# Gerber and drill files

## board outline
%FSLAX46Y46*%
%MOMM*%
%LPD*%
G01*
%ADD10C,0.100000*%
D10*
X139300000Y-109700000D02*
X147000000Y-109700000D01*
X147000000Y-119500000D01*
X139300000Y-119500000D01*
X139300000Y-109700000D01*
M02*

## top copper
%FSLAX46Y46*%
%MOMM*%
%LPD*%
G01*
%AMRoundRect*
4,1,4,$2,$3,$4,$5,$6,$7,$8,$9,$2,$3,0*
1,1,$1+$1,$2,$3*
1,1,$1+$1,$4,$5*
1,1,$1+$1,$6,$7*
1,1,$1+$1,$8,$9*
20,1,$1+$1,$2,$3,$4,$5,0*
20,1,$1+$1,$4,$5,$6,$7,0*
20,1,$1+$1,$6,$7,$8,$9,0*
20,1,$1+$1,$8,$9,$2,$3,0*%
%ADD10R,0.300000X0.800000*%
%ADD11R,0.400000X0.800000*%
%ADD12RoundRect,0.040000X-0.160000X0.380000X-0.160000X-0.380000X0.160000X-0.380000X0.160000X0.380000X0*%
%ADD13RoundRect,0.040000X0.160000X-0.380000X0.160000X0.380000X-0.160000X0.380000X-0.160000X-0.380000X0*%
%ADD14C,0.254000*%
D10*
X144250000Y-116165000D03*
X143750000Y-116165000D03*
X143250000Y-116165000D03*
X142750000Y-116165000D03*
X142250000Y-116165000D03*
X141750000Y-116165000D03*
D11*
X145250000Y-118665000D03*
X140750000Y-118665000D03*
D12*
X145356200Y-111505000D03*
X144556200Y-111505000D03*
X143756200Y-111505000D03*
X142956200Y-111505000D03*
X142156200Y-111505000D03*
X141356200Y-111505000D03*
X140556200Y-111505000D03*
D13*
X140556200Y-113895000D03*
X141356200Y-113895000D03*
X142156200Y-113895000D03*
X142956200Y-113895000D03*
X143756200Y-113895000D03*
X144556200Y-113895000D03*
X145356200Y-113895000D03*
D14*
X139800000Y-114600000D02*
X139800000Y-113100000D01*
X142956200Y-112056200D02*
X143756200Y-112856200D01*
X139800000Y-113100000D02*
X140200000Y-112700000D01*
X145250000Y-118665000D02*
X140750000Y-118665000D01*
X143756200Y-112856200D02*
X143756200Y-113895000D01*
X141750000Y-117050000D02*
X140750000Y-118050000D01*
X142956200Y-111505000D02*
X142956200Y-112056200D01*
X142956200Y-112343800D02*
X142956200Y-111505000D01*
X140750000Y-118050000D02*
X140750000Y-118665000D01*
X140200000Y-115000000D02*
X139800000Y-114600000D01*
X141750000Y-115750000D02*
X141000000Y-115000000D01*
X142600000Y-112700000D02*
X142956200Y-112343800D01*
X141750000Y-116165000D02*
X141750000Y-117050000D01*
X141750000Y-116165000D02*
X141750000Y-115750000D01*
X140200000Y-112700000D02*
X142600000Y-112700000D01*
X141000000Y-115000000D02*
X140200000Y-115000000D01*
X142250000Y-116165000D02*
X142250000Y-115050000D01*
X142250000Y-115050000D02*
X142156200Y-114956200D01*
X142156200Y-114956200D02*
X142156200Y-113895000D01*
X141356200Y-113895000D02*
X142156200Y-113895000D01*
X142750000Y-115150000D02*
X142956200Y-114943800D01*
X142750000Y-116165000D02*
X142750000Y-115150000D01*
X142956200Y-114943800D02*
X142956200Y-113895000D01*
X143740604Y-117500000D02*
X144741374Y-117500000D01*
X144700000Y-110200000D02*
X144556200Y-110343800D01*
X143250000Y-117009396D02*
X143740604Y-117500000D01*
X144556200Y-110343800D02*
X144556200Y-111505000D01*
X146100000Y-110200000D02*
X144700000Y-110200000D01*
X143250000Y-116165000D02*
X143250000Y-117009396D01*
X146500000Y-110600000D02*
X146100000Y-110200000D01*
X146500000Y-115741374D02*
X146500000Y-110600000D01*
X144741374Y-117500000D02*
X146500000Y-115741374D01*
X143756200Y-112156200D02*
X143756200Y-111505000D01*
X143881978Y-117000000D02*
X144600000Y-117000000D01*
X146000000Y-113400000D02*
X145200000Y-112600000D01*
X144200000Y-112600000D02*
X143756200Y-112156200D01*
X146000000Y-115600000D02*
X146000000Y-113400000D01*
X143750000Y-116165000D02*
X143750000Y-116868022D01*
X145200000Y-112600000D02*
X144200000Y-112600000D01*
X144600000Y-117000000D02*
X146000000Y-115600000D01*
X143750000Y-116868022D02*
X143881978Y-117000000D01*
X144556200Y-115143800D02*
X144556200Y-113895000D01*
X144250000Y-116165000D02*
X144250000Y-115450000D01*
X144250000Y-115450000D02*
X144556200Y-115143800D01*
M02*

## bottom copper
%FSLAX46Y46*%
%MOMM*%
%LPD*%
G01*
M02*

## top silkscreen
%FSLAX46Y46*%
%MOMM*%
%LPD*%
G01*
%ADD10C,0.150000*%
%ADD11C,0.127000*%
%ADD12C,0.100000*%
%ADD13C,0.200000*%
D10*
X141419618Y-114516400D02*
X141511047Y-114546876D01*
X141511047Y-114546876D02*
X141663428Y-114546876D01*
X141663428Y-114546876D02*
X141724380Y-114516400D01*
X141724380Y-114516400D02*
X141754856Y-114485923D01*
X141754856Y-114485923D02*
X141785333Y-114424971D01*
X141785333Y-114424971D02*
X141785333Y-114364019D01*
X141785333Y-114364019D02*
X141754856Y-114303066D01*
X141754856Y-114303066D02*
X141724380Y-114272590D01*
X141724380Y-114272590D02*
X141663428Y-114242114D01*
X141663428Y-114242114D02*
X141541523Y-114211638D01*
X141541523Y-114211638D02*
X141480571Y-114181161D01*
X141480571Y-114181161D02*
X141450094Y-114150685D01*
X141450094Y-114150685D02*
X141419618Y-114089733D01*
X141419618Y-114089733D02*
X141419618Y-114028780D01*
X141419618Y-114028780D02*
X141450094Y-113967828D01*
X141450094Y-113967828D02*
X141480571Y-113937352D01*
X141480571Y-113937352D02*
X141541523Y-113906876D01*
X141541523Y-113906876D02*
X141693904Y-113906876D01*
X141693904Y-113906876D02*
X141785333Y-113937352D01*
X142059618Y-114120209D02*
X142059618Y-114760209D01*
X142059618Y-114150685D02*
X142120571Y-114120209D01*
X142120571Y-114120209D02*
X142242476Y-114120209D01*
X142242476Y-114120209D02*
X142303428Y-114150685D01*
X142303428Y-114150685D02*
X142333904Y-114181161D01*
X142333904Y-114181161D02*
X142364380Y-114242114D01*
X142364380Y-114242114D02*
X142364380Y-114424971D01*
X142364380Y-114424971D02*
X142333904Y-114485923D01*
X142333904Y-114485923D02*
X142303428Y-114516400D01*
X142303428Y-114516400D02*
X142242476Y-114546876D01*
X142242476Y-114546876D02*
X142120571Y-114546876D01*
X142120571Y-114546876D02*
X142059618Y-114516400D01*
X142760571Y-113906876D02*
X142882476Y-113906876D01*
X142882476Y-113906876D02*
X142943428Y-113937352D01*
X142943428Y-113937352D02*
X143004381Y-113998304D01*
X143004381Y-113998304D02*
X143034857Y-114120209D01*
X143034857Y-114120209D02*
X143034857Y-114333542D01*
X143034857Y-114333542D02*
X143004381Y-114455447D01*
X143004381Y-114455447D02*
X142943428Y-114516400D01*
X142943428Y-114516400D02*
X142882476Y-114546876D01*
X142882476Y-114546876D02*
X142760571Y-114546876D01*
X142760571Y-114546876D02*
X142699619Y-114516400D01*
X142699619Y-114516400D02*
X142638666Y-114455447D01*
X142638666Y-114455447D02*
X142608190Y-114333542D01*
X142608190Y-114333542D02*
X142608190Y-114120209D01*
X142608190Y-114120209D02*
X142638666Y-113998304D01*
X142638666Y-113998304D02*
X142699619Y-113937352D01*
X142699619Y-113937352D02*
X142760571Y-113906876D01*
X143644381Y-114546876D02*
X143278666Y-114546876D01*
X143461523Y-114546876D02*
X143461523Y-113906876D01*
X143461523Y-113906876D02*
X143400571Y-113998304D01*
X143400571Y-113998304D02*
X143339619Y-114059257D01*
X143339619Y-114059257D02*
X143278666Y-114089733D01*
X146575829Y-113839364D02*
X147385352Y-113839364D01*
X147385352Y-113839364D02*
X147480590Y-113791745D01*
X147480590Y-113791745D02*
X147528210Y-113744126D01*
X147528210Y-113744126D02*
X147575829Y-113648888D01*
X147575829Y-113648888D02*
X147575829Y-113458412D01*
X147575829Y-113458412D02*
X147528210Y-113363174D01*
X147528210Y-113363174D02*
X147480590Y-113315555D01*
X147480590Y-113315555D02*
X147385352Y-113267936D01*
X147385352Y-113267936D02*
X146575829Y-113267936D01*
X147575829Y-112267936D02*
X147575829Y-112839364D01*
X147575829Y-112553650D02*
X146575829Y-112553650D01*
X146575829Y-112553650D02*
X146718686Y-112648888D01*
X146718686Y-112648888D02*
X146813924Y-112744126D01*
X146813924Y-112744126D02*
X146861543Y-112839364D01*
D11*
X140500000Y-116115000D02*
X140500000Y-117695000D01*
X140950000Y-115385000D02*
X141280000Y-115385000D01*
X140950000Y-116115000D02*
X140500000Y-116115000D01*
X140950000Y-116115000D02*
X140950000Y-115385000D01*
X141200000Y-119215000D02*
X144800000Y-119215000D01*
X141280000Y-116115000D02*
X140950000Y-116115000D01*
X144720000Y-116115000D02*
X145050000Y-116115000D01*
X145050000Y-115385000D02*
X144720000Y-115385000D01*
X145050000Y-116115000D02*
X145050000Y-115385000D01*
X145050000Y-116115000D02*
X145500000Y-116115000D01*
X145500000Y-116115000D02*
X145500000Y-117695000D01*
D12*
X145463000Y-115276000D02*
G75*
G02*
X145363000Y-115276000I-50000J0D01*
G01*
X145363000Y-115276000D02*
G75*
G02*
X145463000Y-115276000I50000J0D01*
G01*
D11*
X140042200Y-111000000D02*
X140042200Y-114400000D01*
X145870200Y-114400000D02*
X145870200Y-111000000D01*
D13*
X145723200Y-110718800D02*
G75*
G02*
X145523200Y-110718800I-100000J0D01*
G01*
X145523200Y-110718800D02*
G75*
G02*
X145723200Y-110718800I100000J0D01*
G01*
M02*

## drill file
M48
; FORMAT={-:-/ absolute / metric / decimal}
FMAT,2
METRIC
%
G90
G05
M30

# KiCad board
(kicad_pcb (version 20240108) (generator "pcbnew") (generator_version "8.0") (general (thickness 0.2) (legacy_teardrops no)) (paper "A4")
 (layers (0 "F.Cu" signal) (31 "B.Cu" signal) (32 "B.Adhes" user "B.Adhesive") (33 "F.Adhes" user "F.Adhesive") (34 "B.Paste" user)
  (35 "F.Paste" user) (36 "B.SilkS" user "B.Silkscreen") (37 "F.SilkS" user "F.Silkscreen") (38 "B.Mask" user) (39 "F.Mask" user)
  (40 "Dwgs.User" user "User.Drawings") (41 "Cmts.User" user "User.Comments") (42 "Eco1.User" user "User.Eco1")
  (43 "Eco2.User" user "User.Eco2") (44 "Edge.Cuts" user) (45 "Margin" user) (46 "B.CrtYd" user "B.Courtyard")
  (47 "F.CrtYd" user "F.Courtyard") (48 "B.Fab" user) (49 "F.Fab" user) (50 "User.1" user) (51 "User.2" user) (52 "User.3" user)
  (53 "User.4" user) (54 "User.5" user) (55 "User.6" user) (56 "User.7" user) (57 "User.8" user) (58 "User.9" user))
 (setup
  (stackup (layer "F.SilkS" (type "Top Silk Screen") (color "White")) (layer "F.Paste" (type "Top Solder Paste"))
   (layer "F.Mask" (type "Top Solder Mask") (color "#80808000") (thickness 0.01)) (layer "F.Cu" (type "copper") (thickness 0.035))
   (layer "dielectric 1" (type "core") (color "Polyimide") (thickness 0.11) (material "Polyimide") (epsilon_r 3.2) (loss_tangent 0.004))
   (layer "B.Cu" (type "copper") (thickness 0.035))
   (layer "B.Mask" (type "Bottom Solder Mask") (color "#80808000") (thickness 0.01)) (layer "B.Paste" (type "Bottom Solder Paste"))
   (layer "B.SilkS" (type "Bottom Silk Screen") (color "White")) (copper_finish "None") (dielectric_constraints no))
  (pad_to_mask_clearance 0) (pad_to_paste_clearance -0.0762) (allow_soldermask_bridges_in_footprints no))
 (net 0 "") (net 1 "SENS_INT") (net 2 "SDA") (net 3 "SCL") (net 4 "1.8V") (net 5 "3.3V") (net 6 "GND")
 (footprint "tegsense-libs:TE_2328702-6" (layer "F.Cu") (at 143 116.165)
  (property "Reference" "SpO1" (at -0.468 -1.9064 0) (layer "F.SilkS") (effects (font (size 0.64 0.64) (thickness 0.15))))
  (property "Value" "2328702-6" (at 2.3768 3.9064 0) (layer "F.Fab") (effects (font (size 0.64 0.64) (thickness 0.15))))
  (fp_line (start -2.5 -0.05) (end -2.5 1.53) (stroke (width 0.127) (type solid)) (layer "F.SilkS"))
  (fp_line (start -2.05 -0.78) (end -1.72 -0.78) (stroke (width 0.127) (type solid)) (layer "F.SilkS"))
  (fp_line (start -2.05 -0.05) (end -2.5 -0.05) (stroke (width 0.127) (type solid)) (layer "F.SilkS"))
  (fp_line (start -2.05 -0.05) (end -2.05 -0.78) (stroke (width 0.127) (type solid)) (layer "F.SilkS"))
  (fp_line (start -1.8 3.05) (end 1.8 3.05) (stroke (width 0.127) (type solid)) (layer "F.SilkS"))
  (fp_line (start -1.72 -0.05) (end -2.05 -0.05) (stroke (width 0.127) (type solid)) (layer "F.SilkS"))
  (fp_line (start 1.72 -0.05) (end 2.05 -0.05) (stroke (width 0.127) (type solid)) (layer "F.SilkS"))
  (fp_line (start 2.05 -0.78) (end 1.72 -0.78) (stroke (width 0.127) (type solid)) (layer "F.SilkS"))
  (fp_line (start 2.05 -0.05) (end 2.05 -0.78) (stroke (width 0.127) (type solid)) (layer "F.SilkS"))
  (fp_line (start 2.05 -0.05) (end 2.5 -0.05) (stroke (width 0.127) (type solid)) (layer "F.SilkS"))
  (fp_line (start 2.5 -0.05) (end 2.5 1.53) (stroke (width 0.127) (type solid)) (layer "F.SilkS"))
  (fp_circle (center 2.413 -0.889) (end 2.463 -0.889) (stroke (width 0.1) (type solid)) (fill none) (layer "F.SilkS"))
  (pad "1" smd rect (at 1.25 0 180) (size 0.3 0.8) (layers "F.Cu" "F.Paste" "F.Mask") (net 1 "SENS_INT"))
  (pad "2" smd rect (at 0.75 0 180) (size 0.3 0.8) (layers "F.Cu" "F.Paste" "F.Mask") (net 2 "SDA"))
  (pad "3" smd rect (at 0.25 0 180) (size 0.3 0.8) (layers "F.Cu" "F.Paste" "F.Mask") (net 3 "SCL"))
  (pad "4" smd rect (at -0.25 0 180) (size 0.3 0.8) (layers "F.Cu" "F.Paste" "F.Mask") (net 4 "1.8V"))
  (pad "5" smd rect (at -0.75 0 180) (size 0.3 0.8) (layers "F.Cu" "F.Paste" "F.Mask") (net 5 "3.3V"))
  (pad "6" smd rect (at -1.25 0 180) (size 0.3 0.8) (layers "F.Cu" "F.Paste" "F.Mask") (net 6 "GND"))
  (pad "S1" smd rect (at 2.25 2.5) (size 0.4 0.8) (layers "F.Cu" "F.Paste" "F.Mask") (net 6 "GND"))
  (pad "S2" smd rect (at -2.25 2.5) (size 0.4 0.8) (layers "F.Cu" "F.Paste" "F.Mask") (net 6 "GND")))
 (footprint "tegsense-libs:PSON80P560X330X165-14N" (layer "F.Cu") (at 142.9562 112.7 -90)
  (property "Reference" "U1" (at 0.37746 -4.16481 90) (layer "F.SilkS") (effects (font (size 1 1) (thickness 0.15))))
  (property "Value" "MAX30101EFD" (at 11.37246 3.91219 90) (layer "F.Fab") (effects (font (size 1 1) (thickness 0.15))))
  (fp_line (start -1.7 2.914) (end 1.7 2.914) (stroke (width 0.127) (type solid)) (layer "F.SilkS"))
  (fp_line (start 1.7 -2.914) (end -1.7 -2.914) (stroke (width 0.127) (type solid)) (layer "F.SilkS"))
  (fp_circle (center -1.9812 -2.667) (end -1.8812 -2.667) (stroke (width 0.2) (type solid)) (fill none) (layer "F.SilkS"))
  (pad "1" smd roundrect (at -1.195 -2.4 270) (size 0.84 0.4) (layers "F.Cu" "F.Paste" "F.Mask") (roundrect_rratio 0.1))
  (pad "2" smd roundrect (at -1.195 -1.6 270) (size 0.84 0.4) (layers "F.Cu" "F.Paste" "F.Mask") (roundrect_rratio 0.1) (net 3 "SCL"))
  (pad "3" smd roundrect (at -1.195 -0.8 270) (size 0.84 0.4) (layers "F.Cu" "F.Paste" "F.Mask") (roundrect_rratio 0.1) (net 2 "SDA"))
  (pad "4" smd roundrect (at -1.195 0 270) (size 0.84 0.4) (layers "F.Cu" "F.Paste" "F.Mask") (roundrect_rratio 0.1) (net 6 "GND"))
  (pad "5" smd roundrect (at -1.195 0.8 270) (size 0.84 0.4) (layers "F.Cu" "F.Paste" "F.Mask") (roundrect_rratio 0.1))
  (pad "6" smd roundrect (at -1.195 1.6 270) (size 0.84 0.4) (layers "F.Cu" "F.Paste" "F.Mask") (roundrect_rratio 0.1))
  (pad "7" smd roundrect (at -1.195 2.4 270) (size 0.84 0.4) (layers "F.Cu" "F.Paste" "F.Mask") (roundrect_rratio 0.1))
  (pad "8" smd roundrect (at 1.195 2.4 90) (size 0.84 0.4) (layers "F.Cu" "F.Paste" "F.Mask") (roundrect_rratio 0.1))
  (pad "9" smd roundrect (at 1.195 1.6 90) (size 0.84 0.4) (layers "F.Cu" "F.Paste" "F.Mask") (roundrect_rratio 0.1) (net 5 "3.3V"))
  (pad "10" smd roundrect (at 1.195 0.8 90) (size 0.84 0.4) (layers "F.Cu" "F.Paste" "F.Mask") (roundrect_rratio 0.1) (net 5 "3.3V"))
  (pad "11" smd roundrect (at 1.195 0 90) (size 0.84 0.4) (layers "F.Cu" "F.Paste" "F.Mask") (roundrect_rratio 0.1) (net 4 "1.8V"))
  (pad "12" smd roundrect (at 1.195 -0.8 90) (size 0.84 0.4) (layers "F.Cu" "F.Paste" "F.Mask") (roundrect_rratio 0.1) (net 6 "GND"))
  (pad "13" smd roundrect (at 1.195 -1.6 90) (size 0.84 0.4) (layers "F.Cu" "F.Paste" "F.Mask") (roundrect_rratio 0.1) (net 1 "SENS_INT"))
  (pad "14" smd roundrect (at 1.195 -2.4 90) (size 0.84 0.4) (layers "F.Cu" "F.Paste" "F.Mask") (roundrect_rratio 0.1)))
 (gr_rect (start 139.3 109.7) (end 147 119.5) (stroke (width 0.1) (type solid)) (fill none) (layer "Edge.Cuts"))
 (segment (start 139.8 114.6) (end 139.8 113.1) (width 0.254) (layer "F.Cu") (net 6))
 (segment (start 142.9562 112.0562) (end 143.7562 112.8562) (width 0.254) (layer "F.Cu") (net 6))
 (segment (start 139.8 113.1) (end 140.2 112.7) (width 0.254) (layer "F.Cu") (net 6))
 (segment (start 145.25 118.665) (end 140.75 118.665) (width 0.254) (layer "F.Cu") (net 6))
 (segment (start 143.7562 112.8562) (end 143.7562 113.895) (width 0.254) (layer "F.Cu") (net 6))
 (segment (start 141.75 117.05) (end 140.75 118.05) (width 0.254) (layer "F.Cu") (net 6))
 (segment (start 142.9562 111.505) (end 142.9562 112.0562) (width 0.254) (layer "F.Cu") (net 6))
 (segment (start 142.9562 112.3438) (end 142.9562 111.505) (width 0.254) (layer "F.Cu") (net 6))
 (segment (start 140.75 118.05) (end 140.75 118.665) (width 0.254) (layer "F.Cu") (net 6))
 (segment (start 140.2 115) (end 139.8 114.6) (width 0.254) (layer "F.Cu") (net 6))
 (segment (start 141.75 115.75) (end 141 115) (width 0.254) (layer "F.Cu") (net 6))
 (segment (start 142.6 112.7) (end 142.9562 112.3438) (width 0.254) (layer "F.Cu") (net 6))
 (segment (start 141.75 116.165) (end 141.75 117.05) (width 0.254) (layer "F.Cu") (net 6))
 (segment (start 141.75 116.165) (end 141.75 115.75) (width 0.254) (layer "F.Cu") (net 6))
 (segment (start 140.2 112.7) (end 142.6 112.7) (width 0.254) (layer "F.Cu") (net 6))
 (segment (start 141 115) (end 140.2 115) (width 0.254) (layer "F.Cu") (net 6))
 (segment (start 142.25 116.165) (end 142.25 115.05) (width 0.254) (layer "F.Cu") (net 5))
 (segment (start 142.25 115.05) (end 142.1562 114.9562) (width 0.254) (layer "F.Cu") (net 5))
 (segment (start 142.1562 114.9562) (end 142.1562 113.895) (width 0.254) (layer "F.Cu") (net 5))
 (segment (start 141.3562 113.895) (end 142.1562 113.895) (width 0.254) (layer "F.Cu") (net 5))
 (segment (start 142.75 115.15) (end 142.9562 114.9438) (width 0.254) (layer "F.Cu") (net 4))
 (segment (start 142.75 116.165) (end 142.75 115.15) (width 0.254) (layer "F.Cu") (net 4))
 (segment (start 142.9562 114.9438) (end 142.9562 113.895) (width 0.254) (layer "F.Cu") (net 4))
 (segment (start 143.740604 117.5) (end 144.741374 117.5) (width 0.254) (layer "F.Cu") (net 3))
 (segment (start 144.7 110.2) (end 144.5562 110.3438) (width 0.254) (layer "F.Cu") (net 3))
 (segment (start 143.25 117.009396) (end 143.740604 117.5) (width 0.254) (layer "F.Cu") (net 3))
 (segment (start 144.5562 110.3438) (end 144.5562 111.505) (width 0.254) (layer "F.Cu") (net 3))
 (segment (start 146.1 110.2) (end 144.7 110.2) (width 0.254) (layer "F.Cu") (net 3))
 (segment (start 143.25 116.165) (end 143.25 117.009396) (width 0.254) (layer "F.Cu") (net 3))
 (segment (start 146.5 110.6) (end 146.1 110.2) (width 0.254) (layer "F.Cu") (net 3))
 (segment (start 146.5 115.741374) (end 146.5 110.6) (width 0.254) (layer "F.Cu") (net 3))
 (segment (start 144.741374 117.5) (end 146.5 115.741374) (width 0.254) (layer "F.Cu") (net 3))
 (segment (start 143.7562 112.1562) (end 143.7562 111.505) (width 0.254) (layer "F.Cu") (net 2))
 (segment (start 143.881978 117) (end 144.6 117) (width 0.254) (layer "F.Cu") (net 2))
 (segment (start 146 113.4) (end 145.2 112.6) (width 0.254) (layer "F.Cu") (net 2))
 (segment (start 144.2 112.6) (end 143.7562 112.1562) (width 0.254) (layer "F.Cu") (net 2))
 (segment (start 146 115.6) (end 146 113.4) (width 0.254) (layer "F.Cu") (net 2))
 (segment (start 143.75 116.165) (end 143.75 116.868022) (width 0.254) (layer "F.Cu") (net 2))
 (segment (start 145.2 112.6) (end 144.2 112.6) (width 0.254) (layer "F.Cu") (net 2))
 (segment (start 144.6 117) (end 146 115.6) (width 0.254) (layer "F.Cu") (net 2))
 (segment (start 143.75 116.868022) (end 143.881978 117) (width 0.254) (layer "F.Cu") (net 2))
 (segment (start 144.5562 115.1438) (end 144.5562 113.895) (width 0.254) (layer "F.Cu") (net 1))
 (segment (start 144.25 116.165) (end 144.25 115.45) (width 0.254) (layer "F.Cu") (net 1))
 (segment (start 144.25 115.45) (end 144.5562 115.1438) (width 0.254) (layer "F.Cu") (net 1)))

